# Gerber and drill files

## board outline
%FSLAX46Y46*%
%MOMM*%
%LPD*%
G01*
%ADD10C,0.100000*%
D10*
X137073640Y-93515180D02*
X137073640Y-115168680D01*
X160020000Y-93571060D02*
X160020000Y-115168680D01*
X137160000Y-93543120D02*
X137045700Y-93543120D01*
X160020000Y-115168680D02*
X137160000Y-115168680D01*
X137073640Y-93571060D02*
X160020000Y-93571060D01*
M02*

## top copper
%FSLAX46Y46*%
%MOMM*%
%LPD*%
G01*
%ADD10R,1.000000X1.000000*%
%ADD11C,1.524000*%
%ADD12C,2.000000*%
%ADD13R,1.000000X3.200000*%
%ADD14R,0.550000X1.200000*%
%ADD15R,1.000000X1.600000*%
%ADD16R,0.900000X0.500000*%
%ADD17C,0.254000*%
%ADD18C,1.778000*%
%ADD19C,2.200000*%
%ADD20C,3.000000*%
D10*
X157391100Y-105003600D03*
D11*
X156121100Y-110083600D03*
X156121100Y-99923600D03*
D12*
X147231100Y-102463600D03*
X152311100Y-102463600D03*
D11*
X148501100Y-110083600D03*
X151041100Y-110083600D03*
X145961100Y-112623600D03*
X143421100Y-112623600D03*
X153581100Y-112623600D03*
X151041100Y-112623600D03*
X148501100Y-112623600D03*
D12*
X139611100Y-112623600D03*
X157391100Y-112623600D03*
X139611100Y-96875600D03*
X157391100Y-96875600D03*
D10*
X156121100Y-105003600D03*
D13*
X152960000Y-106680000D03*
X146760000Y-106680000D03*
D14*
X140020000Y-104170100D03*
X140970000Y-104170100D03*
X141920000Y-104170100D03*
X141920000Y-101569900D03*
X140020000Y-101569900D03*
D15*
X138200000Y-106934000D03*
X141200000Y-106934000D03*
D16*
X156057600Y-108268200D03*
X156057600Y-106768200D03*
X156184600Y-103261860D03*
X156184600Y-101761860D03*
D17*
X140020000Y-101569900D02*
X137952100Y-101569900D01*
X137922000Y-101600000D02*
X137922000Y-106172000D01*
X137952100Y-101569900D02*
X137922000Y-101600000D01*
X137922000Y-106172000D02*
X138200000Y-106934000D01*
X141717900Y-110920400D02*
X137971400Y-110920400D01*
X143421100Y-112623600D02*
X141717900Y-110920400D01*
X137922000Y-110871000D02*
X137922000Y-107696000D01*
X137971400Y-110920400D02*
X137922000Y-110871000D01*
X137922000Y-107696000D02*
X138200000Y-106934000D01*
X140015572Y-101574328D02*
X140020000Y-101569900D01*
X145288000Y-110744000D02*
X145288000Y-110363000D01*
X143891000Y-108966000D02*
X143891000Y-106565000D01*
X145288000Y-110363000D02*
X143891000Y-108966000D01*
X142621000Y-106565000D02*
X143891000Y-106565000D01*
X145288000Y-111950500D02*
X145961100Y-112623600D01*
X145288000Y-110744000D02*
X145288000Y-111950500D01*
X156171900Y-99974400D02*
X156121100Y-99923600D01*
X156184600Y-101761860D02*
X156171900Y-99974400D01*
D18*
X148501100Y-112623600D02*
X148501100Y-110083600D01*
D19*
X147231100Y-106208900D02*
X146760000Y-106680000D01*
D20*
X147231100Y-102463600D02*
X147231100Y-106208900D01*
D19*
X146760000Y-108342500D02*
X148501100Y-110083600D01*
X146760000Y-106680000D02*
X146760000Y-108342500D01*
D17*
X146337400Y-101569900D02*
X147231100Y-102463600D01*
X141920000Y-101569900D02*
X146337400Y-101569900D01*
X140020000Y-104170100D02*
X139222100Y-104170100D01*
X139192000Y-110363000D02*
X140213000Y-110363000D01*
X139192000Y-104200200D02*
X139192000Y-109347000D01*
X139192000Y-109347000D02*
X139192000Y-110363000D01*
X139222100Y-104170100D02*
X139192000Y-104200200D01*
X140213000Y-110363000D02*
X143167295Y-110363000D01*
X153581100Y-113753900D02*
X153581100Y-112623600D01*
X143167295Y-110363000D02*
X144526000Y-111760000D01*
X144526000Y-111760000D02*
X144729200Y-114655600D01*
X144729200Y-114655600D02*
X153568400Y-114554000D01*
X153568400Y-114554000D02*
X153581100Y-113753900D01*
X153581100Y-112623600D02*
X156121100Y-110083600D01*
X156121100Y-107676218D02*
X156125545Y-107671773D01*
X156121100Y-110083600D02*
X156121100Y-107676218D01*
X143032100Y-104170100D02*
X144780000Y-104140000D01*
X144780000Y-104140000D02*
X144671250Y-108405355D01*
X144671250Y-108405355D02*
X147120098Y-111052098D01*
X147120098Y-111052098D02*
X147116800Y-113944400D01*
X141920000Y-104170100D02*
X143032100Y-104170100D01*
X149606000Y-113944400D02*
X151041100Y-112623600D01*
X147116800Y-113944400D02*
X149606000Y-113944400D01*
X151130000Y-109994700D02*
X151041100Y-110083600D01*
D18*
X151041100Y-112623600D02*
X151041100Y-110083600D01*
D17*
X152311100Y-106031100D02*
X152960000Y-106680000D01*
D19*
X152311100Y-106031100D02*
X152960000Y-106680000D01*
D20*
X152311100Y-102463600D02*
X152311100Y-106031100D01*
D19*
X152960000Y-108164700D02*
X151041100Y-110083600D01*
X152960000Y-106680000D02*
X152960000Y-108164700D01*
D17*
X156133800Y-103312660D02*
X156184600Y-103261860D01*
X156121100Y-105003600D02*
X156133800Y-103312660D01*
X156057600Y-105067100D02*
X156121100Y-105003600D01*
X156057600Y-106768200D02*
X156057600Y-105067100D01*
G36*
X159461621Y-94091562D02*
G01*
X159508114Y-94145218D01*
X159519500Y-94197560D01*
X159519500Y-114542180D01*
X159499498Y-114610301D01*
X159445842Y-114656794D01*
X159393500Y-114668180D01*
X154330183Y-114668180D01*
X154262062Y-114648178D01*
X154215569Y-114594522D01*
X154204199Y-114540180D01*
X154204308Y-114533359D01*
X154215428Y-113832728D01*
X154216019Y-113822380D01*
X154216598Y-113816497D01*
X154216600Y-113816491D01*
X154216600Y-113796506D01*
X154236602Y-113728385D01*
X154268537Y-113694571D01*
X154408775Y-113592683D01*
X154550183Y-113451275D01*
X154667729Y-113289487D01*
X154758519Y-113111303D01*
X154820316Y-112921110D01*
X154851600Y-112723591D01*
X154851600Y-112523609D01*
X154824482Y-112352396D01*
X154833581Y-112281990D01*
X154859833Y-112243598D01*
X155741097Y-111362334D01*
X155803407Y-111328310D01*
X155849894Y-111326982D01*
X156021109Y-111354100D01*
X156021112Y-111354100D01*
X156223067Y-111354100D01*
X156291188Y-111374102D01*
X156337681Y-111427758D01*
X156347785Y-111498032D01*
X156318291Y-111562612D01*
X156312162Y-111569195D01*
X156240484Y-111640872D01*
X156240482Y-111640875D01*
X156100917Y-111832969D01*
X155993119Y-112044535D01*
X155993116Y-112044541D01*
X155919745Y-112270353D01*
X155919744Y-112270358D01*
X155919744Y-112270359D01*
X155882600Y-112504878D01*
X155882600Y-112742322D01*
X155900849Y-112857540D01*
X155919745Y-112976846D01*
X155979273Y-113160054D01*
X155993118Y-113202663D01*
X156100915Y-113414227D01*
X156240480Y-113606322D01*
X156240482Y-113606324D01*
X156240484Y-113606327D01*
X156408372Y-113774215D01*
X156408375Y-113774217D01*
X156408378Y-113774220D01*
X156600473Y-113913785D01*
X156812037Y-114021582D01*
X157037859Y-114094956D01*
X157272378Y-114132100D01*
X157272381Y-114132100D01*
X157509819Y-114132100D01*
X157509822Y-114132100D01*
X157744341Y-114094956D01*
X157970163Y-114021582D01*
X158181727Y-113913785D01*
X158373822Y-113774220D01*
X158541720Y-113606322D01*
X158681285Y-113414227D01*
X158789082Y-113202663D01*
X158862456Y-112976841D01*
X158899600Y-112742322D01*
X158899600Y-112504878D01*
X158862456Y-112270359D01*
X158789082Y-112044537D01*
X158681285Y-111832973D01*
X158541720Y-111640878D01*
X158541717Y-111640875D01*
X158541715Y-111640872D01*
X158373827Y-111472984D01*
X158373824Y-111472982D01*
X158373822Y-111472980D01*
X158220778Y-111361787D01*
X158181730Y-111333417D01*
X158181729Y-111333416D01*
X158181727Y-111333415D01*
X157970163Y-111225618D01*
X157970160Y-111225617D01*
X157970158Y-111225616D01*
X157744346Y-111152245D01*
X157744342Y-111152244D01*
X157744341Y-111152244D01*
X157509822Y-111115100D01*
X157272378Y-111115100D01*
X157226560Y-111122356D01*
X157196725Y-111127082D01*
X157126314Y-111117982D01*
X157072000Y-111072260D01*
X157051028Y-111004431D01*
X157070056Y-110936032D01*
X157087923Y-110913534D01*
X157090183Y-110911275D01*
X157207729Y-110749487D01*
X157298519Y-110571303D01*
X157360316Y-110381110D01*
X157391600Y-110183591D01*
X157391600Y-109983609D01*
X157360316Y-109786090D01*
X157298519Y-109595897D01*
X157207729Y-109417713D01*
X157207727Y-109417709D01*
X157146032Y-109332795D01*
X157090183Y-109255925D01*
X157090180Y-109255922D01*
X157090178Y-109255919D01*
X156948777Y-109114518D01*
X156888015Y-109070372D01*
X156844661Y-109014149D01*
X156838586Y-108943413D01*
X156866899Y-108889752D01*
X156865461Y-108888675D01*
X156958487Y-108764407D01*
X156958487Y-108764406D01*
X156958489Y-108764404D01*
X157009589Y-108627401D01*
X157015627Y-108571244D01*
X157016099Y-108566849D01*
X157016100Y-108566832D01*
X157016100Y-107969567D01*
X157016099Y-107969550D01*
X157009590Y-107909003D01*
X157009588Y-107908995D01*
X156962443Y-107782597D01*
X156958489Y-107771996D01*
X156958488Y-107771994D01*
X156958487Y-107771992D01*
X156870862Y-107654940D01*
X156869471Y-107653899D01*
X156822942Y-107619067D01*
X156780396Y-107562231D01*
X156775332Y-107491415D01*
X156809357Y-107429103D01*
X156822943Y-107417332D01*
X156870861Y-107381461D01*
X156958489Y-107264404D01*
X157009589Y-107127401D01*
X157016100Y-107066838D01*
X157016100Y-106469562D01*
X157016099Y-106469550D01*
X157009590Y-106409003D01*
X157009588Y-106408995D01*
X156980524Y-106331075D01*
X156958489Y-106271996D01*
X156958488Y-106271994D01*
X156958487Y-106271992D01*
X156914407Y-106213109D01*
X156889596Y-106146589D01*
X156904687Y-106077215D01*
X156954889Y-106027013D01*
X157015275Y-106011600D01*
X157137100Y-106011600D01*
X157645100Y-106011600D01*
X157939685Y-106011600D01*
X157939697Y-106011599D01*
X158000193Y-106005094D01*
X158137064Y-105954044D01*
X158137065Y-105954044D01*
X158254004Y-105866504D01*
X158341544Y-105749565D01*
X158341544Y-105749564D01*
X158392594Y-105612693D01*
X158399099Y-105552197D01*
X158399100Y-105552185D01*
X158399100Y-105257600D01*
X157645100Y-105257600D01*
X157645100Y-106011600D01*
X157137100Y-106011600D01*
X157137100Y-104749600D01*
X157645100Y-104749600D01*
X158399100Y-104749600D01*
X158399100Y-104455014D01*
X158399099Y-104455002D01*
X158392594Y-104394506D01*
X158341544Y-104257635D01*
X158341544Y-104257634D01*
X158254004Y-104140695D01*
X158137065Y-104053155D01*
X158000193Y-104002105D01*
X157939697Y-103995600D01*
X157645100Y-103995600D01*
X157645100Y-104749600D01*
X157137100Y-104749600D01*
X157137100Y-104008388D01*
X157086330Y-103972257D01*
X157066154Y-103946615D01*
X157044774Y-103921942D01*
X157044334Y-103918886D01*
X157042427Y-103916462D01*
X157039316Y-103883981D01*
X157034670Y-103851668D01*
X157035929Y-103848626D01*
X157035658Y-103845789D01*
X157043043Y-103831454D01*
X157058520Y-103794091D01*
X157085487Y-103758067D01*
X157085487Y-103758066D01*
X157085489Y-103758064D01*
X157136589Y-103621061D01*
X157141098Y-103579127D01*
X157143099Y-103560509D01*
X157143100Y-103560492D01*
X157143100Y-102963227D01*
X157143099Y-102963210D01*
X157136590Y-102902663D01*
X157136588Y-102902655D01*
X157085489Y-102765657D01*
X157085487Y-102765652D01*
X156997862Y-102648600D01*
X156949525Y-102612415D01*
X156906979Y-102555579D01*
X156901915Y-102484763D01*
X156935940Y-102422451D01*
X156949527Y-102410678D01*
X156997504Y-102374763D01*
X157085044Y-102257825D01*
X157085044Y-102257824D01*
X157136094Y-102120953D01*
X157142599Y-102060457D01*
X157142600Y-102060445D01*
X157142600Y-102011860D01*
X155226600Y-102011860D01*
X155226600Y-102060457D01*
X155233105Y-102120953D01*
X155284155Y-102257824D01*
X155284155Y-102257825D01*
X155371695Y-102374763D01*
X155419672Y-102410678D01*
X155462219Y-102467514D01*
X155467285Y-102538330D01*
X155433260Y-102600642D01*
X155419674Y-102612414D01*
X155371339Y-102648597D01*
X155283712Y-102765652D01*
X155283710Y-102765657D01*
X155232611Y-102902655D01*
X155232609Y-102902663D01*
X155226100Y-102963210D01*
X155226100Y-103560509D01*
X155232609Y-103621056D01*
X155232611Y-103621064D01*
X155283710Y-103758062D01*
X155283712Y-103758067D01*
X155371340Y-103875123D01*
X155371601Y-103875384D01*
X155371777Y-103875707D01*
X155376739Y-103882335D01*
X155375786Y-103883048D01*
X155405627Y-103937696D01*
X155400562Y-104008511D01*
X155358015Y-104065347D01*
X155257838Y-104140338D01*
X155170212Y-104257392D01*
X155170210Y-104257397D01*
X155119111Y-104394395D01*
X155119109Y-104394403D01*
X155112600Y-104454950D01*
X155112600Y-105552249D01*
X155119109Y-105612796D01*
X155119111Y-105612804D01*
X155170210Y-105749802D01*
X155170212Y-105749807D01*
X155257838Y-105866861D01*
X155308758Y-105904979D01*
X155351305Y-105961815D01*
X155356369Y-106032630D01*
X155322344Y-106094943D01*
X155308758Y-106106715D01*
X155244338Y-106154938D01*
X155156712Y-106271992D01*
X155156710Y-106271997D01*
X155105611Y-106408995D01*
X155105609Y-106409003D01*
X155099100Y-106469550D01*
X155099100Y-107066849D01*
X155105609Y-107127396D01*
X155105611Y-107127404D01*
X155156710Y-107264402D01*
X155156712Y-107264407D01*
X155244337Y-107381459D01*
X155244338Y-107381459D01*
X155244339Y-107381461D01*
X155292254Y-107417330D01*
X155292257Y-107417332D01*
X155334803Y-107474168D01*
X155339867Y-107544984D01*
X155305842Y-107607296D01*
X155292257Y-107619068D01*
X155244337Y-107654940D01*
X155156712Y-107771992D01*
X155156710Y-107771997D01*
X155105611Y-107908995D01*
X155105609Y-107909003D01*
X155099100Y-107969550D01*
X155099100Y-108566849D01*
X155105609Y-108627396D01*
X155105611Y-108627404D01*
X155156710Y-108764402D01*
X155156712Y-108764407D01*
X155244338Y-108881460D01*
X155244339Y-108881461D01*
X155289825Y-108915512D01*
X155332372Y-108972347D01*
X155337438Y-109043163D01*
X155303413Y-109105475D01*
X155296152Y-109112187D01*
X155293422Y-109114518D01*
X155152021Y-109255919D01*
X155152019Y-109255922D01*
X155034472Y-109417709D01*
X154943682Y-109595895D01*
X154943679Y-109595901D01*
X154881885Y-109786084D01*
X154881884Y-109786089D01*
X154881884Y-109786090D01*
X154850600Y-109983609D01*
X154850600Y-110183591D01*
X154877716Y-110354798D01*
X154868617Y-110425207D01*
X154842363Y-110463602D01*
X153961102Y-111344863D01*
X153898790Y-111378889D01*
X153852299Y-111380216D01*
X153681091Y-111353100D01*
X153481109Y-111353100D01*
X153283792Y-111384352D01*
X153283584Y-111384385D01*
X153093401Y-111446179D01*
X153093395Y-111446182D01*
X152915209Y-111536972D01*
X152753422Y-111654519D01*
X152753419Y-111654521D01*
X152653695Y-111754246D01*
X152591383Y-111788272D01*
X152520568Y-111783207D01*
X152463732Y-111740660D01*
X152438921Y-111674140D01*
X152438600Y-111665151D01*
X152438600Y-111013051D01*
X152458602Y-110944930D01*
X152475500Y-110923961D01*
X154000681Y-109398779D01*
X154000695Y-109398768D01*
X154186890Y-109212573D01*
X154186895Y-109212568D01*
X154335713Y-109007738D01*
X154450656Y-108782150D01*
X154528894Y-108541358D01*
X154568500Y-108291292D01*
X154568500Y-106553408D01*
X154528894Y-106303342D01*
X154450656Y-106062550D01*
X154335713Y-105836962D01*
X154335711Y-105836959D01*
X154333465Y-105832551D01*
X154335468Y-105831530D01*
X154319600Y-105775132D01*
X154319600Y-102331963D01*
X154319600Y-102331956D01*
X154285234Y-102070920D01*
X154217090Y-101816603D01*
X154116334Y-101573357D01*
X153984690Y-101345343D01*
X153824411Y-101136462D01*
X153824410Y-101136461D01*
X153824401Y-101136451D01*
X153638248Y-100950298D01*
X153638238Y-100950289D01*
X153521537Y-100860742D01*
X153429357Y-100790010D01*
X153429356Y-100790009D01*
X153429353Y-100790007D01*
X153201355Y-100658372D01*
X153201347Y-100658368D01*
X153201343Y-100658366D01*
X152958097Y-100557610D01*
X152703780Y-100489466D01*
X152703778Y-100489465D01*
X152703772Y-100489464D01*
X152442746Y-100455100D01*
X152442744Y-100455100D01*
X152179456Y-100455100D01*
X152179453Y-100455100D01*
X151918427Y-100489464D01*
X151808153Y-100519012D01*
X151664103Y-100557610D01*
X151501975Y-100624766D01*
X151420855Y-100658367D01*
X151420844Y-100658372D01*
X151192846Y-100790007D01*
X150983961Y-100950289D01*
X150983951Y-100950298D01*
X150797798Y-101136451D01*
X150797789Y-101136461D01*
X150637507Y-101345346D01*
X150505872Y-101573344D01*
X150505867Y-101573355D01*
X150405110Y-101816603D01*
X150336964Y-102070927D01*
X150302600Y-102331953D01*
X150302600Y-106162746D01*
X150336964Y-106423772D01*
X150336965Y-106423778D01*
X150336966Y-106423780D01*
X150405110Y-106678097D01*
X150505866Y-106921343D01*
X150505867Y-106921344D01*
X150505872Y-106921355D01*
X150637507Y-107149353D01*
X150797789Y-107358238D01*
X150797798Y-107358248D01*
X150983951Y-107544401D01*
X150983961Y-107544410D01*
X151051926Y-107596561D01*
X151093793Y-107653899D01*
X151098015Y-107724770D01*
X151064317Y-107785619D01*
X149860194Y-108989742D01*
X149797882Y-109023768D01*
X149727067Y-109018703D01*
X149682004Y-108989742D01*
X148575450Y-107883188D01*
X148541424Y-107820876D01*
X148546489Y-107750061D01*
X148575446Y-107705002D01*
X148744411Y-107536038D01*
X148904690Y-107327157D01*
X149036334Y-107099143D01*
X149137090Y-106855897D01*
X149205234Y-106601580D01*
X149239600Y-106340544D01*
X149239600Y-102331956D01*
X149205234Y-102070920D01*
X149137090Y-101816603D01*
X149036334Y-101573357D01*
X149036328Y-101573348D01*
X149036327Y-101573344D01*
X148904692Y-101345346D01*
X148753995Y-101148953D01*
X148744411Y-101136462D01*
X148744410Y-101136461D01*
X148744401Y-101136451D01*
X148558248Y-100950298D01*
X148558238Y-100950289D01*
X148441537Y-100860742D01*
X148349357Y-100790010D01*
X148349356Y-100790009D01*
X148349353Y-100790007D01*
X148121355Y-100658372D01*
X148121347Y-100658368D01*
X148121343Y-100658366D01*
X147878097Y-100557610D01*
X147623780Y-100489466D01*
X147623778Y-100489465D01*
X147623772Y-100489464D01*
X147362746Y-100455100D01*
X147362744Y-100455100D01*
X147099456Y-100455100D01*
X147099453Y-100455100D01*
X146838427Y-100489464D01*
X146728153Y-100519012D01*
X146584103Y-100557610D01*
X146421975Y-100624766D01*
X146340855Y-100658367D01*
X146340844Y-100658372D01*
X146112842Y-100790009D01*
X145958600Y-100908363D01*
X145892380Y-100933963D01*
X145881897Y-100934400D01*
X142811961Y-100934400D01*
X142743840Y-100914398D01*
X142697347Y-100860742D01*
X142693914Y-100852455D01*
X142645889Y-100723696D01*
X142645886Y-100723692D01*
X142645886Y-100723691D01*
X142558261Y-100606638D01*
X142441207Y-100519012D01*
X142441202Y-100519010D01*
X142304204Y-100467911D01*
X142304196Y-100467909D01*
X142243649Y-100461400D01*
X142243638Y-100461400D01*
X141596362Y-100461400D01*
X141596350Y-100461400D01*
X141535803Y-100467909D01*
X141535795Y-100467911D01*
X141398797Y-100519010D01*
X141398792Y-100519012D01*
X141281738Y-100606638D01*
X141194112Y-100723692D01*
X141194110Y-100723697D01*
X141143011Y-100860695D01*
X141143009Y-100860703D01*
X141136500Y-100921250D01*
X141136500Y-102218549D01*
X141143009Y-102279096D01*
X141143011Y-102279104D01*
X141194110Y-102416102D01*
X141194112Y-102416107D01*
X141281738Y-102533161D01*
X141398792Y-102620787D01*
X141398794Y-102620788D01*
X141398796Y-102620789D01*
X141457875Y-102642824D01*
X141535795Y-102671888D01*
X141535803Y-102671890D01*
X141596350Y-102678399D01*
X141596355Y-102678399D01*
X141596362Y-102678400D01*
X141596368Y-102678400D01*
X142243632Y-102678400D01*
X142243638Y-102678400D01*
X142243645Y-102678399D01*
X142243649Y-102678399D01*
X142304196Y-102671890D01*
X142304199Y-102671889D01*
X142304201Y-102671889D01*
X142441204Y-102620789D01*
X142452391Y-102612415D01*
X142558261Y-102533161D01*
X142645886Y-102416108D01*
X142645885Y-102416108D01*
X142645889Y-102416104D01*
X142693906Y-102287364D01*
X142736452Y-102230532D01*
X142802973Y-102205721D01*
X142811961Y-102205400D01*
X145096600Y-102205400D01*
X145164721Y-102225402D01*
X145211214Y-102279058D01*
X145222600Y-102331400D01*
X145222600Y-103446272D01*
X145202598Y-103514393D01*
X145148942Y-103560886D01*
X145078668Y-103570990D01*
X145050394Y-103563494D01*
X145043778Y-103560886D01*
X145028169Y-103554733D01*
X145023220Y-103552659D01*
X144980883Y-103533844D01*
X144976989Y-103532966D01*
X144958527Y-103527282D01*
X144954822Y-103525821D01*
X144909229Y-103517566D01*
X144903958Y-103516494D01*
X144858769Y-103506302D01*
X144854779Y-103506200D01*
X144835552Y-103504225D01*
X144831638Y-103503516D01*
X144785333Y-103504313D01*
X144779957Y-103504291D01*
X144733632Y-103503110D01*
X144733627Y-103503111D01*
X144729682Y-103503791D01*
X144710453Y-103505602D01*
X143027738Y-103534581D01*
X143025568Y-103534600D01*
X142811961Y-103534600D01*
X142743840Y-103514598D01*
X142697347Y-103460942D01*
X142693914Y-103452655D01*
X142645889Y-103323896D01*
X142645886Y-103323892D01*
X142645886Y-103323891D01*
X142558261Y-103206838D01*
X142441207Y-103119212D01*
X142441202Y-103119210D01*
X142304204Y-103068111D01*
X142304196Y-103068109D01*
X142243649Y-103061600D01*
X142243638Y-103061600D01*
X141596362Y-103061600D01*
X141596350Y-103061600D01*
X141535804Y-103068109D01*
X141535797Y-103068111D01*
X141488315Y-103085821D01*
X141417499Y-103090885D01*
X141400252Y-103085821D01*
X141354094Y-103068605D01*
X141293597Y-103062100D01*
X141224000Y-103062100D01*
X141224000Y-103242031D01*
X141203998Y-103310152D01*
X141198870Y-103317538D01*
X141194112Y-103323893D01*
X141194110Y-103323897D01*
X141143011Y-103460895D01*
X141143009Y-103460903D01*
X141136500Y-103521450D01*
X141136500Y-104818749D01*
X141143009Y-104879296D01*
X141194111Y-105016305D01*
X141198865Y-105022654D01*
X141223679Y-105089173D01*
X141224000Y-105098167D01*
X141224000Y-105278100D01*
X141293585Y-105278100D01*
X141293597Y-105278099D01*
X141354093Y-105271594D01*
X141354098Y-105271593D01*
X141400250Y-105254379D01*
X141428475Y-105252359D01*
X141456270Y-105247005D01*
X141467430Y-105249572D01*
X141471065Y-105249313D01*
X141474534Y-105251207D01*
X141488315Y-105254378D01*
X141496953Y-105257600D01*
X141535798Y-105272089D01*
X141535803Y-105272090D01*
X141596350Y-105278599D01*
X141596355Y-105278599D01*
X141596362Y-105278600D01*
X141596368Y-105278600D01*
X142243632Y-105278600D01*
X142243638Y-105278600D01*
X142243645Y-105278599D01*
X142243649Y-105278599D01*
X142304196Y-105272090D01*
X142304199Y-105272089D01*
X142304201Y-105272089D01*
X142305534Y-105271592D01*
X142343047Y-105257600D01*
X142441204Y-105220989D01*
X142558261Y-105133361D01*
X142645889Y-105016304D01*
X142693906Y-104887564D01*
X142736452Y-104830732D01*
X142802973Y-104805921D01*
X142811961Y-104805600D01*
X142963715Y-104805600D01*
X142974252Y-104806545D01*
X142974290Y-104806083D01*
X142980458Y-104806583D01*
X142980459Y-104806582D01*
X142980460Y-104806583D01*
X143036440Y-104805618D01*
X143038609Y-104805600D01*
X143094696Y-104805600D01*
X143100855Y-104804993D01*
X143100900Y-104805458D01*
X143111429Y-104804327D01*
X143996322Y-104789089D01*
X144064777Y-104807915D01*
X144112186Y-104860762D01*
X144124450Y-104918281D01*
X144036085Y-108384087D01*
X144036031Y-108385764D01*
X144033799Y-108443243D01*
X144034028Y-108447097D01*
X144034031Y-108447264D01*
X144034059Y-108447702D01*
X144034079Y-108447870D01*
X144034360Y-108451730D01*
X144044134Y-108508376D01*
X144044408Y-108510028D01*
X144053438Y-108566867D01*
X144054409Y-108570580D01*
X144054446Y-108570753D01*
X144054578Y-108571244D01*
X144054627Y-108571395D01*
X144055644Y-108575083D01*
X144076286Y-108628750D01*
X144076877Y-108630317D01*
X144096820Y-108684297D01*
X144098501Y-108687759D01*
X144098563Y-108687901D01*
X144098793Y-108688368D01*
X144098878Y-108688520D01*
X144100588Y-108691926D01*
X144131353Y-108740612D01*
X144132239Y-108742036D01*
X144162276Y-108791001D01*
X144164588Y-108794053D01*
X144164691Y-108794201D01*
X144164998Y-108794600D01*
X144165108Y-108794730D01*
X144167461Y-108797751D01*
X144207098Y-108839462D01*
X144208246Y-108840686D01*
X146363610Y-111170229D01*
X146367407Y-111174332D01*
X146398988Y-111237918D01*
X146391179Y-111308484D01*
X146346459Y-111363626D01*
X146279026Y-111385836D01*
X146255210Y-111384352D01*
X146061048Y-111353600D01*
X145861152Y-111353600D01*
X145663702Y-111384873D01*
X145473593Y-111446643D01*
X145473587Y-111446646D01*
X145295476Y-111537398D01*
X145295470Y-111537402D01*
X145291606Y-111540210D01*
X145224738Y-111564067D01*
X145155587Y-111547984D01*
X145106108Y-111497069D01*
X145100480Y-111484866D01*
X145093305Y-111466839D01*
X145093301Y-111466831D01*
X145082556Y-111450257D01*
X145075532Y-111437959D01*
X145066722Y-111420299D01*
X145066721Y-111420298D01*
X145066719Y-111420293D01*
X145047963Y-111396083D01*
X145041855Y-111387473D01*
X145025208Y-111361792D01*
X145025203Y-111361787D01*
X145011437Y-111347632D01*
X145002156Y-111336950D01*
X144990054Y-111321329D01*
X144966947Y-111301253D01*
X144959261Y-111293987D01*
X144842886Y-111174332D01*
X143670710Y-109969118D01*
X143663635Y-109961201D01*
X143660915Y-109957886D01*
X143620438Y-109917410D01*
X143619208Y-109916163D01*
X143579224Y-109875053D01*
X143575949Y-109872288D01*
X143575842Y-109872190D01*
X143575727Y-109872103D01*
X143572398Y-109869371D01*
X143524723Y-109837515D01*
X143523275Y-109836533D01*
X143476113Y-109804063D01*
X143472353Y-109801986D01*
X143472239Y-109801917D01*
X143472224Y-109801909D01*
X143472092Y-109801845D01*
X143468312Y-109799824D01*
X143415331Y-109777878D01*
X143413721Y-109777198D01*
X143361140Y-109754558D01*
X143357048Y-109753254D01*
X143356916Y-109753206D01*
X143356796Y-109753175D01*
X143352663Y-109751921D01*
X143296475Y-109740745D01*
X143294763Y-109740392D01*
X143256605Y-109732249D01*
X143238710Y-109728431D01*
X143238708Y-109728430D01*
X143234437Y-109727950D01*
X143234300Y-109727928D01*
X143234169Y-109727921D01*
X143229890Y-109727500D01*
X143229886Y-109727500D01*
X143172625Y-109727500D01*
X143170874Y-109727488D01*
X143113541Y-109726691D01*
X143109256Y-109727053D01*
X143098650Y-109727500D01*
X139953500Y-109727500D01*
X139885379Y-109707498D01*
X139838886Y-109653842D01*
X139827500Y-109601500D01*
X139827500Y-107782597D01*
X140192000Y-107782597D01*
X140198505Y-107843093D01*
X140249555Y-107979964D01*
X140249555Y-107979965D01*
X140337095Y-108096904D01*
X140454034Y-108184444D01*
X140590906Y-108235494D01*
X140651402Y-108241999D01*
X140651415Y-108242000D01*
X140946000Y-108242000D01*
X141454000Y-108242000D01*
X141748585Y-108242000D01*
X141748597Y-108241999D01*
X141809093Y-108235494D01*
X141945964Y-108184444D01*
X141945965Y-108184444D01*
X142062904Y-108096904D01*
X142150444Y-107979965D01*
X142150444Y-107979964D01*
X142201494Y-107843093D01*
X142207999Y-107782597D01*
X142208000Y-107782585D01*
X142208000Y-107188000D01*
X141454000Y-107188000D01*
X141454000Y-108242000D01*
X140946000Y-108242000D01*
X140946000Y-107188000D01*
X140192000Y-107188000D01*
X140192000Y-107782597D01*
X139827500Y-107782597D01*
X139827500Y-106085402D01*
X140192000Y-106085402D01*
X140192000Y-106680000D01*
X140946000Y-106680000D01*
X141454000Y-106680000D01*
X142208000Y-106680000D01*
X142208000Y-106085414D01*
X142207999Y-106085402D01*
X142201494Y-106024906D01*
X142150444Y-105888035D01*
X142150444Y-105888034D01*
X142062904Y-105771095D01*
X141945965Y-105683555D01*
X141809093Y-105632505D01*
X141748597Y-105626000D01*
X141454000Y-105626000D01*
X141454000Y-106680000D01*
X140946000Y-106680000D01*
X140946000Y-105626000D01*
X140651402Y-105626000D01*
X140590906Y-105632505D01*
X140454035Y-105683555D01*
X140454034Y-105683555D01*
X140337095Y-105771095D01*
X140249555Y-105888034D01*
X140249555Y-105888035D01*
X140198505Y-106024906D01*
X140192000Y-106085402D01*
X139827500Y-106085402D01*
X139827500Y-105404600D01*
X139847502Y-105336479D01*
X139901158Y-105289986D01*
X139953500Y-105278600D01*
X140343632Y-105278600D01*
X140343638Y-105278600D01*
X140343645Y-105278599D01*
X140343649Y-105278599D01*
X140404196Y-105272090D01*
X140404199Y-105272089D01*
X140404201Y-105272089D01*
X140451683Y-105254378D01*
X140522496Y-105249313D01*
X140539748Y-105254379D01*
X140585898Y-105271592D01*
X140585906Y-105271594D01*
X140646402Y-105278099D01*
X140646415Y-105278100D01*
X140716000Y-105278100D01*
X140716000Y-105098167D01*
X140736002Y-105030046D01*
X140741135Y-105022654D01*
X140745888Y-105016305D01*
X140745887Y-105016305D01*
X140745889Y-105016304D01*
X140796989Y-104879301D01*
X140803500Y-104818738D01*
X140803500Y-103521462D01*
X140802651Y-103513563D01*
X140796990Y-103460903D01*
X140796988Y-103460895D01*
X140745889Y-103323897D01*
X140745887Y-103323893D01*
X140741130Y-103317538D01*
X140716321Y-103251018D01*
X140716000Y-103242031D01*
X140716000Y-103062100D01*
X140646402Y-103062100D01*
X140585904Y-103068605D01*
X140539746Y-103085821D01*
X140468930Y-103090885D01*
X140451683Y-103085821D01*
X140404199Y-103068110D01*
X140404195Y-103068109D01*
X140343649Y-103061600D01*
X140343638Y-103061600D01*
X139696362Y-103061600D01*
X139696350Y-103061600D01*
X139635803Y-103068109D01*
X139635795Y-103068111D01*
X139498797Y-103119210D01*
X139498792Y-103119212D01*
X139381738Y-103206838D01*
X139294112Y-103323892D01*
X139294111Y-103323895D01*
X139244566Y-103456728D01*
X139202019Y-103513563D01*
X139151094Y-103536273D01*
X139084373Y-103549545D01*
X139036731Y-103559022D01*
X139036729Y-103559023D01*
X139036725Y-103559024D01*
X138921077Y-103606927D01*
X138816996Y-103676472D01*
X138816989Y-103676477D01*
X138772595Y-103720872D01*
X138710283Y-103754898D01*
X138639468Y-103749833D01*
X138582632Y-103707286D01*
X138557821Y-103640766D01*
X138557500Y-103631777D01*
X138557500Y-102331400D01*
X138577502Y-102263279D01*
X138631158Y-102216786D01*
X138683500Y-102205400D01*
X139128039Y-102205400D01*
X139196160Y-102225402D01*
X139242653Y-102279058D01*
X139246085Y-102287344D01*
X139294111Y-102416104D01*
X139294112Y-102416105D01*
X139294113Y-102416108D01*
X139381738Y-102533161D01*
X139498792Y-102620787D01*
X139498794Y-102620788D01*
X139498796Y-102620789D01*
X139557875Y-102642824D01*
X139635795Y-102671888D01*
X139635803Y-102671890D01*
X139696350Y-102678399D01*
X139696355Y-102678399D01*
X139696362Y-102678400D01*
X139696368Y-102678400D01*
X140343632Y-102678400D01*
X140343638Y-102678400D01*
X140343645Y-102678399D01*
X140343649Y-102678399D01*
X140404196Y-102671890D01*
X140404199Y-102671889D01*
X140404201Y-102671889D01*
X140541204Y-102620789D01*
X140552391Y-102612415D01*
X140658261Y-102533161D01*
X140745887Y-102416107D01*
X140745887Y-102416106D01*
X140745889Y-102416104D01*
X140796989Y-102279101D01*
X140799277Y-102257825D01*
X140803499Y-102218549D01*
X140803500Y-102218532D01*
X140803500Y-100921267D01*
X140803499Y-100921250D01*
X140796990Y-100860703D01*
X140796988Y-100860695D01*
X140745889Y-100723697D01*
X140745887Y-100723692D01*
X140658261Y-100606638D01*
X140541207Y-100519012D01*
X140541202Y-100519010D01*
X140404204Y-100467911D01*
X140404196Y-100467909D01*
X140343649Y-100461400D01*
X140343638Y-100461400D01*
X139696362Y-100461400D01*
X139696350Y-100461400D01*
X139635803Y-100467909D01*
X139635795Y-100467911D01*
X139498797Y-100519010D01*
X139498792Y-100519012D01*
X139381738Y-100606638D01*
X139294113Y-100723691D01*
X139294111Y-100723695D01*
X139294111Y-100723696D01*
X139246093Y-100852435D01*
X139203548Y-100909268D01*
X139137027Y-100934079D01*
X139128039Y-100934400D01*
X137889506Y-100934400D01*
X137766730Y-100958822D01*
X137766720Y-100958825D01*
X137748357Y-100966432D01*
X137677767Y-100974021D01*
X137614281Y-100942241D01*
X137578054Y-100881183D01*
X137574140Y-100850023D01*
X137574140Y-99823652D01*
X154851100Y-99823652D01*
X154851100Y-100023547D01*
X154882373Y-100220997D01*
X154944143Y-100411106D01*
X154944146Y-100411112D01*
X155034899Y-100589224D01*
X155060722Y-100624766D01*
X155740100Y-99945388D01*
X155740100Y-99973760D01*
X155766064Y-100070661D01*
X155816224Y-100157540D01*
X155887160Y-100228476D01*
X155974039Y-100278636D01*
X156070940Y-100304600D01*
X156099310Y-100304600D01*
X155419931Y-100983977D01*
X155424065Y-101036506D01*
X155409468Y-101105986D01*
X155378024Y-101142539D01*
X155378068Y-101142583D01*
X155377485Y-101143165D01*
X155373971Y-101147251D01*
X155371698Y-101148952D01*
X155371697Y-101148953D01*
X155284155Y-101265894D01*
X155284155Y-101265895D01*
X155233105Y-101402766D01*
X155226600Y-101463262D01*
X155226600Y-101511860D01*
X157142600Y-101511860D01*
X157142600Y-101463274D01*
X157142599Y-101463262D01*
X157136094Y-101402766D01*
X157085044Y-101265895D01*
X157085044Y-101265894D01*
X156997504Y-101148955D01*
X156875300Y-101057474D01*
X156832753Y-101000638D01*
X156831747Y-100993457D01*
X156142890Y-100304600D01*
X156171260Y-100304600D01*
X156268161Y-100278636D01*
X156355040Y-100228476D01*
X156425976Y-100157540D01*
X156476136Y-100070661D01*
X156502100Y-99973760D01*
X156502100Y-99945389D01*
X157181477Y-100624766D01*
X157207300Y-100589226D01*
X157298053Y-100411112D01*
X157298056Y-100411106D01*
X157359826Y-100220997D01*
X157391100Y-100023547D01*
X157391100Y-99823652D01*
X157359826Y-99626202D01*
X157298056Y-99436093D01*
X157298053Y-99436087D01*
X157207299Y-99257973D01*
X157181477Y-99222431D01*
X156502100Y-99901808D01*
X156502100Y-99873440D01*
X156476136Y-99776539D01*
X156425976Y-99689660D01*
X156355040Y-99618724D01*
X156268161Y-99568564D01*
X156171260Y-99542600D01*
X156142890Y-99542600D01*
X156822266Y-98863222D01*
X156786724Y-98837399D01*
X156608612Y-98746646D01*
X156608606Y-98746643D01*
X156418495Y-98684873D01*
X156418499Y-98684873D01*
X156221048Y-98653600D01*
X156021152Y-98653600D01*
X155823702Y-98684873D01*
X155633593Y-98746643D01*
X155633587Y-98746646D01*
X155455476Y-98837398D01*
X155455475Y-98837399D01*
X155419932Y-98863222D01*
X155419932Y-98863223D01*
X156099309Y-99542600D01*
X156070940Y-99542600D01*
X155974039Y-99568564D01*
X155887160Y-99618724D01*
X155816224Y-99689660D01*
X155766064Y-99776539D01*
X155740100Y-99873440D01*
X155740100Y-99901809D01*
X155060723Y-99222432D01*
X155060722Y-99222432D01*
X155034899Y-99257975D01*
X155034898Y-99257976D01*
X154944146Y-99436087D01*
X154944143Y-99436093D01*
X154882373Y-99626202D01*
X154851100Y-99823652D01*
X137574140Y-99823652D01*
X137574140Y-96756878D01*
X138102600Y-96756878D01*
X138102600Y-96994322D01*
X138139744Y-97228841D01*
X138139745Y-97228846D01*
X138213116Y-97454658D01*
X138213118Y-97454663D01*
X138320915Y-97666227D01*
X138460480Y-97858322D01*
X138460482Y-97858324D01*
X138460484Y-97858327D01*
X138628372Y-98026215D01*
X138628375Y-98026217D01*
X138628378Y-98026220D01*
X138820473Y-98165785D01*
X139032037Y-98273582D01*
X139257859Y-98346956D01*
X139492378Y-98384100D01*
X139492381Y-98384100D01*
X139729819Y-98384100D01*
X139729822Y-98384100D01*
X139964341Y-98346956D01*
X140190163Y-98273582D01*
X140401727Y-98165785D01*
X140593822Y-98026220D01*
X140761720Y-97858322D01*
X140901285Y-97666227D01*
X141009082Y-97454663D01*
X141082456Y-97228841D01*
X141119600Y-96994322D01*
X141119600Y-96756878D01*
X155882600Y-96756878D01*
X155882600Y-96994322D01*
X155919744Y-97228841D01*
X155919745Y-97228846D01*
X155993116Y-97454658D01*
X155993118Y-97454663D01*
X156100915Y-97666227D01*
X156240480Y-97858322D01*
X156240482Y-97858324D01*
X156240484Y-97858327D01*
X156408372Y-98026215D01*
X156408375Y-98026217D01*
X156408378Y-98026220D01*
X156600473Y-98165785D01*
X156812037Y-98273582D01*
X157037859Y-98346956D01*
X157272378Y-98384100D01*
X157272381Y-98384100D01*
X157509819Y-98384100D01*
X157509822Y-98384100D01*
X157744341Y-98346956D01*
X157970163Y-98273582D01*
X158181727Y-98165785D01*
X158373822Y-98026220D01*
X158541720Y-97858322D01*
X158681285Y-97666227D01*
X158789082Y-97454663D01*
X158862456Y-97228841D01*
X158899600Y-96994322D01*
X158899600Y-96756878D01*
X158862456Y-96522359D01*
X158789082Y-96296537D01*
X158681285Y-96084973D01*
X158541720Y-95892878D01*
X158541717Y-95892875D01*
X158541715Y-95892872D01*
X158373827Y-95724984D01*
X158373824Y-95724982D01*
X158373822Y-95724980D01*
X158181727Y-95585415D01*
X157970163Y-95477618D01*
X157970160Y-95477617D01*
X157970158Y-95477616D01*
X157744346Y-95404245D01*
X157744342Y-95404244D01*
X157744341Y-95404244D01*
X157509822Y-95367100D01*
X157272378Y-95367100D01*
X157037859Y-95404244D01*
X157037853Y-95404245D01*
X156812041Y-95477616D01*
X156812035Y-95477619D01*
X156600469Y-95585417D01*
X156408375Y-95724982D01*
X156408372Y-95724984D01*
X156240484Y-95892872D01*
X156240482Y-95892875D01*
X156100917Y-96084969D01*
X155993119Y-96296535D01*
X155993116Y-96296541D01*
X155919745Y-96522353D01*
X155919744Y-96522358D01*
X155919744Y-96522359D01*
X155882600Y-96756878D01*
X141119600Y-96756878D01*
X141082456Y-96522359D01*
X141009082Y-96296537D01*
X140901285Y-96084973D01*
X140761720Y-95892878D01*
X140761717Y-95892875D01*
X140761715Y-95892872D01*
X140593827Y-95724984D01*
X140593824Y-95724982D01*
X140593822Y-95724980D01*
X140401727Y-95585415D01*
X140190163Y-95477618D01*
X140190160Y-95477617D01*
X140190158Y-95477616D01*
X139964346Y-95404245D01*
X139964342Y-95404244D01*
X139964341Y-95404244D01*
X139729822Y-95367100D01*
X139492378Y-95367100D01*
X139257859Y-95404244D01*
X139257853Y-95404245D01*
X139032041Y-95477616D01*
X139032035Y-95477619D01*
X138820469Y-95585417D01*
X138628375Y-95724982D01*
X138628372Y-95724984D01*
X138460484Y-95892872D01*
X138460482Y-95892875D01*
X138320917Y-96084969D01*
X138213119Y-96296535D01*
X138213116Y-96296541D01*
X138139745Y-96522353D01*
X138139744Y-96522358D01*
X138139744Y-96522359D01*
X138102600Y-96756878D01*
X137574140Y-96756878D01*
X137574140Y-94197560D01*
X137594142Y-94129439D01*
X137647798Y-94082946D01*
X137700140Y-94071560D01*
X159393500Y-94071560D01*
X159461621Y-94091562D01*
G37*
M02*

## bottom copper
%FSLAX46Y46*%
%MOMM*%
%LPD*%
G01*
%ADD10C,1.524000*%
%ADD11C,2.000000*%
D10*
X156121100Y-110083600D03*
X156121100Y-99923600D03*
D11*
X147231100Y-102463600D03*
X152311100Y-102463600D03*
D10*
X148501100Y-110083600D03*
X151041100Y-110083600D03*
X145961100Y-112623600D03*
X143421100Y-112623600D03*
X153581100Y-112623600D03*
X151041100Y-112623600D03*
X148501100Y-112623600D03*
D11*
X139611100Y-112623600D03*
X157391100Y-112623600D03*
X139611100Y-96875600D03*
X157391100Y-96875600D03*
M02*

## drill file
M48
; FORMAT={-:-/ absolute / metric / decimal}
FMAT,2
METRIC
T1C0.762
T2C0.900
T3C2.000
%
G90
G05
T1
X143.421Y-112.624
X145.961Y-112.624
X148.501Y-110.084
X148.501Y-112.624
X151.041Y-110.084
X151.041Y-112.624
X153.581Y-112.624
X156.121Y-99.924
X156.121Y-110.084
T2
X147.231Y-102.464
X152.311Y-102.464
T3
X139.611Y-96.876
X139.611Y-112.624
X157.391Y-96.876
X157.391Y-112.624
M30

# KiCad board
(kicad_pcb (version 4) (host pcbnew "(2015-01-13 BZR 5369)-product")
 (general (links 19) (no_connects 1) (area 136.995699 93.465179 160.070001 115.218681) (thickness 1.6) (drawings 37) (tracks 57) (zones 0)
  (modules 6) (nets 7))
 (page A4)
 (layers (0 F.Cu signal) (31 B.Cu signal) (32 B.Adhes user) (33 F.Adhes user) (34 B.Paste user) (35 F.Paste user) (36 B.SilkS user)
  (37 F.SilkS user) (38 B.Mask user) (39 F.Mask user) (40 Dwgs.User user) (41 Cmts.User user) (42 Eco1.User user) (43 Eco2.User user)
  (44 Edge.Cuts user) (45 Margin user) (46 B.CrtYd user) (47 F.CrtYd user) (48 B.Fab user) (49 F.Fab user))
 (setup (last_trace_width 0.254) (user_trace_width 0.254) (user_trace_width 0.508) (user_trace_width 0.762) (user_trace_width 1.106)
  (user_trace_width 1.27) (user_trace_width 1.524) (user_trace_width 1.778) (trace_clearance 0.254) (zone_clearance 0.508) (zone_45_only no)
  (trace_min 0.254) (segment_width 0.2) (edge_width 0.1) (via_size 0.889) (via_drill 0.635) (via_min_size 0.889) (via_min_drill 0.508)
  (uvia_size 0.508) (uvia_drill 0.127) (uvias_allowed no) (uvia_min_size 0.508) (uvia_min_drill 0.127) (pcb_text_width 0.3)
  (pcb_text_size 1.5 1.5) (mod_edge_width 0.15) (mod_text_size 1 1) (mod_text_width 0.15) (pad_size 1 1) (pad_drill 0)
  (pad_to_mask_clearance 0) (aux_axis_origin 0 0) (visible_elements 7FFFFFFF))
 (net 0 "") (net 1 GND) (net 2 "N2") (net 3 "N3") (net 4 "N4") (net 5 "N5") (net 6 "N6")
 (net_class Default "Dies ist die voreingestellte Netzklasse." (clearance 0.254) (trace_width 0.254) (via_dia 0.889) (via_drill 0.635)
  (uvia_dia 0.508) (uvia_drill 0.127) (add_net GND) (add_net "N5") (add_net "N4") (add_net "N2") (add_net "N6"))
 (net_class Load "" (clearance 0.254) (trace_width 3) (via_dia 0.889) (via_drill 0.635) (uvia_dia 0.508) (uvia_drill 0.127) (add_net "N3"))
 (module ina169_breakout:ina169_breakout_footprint (layer F.Cu) (at 148.5011 105.0036)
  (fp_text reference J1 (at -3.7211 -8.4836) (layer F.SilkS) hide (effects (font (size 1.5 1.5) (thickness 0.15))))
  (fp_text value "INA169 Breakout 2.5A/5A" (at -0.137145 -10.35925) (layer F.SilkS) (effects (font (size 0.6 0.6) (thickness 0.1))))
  (pad 2 smd rect (at 8.89 0) (size 1 1) (layers F.Cu F.Paste F.Mask) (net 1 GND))
  (pad 5 thru_hole circle (at 7.62 5.08) (size 1.524 1.524) (drill 0.762) (layers *.Cu *.Mask F.SilkS) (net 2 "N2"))
  (pad 2 thru_hole circle (at 7.62 -5.08) (size 1.524 1.524) (drill 0.762) (layers *.Cu *.Mask F.SilkS) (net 1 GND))
  (pad 3 thru_hole circle (at -1.27 -2.54) (size 2 2) (drill 0.9) (layers *.Cu *.Mask F.SilkS) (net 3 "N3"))
  (pad 4 thru_hole circle (at 3.81 -2.54) (size 2 2) (drill 0.9) (layers *.Cu *.Mask F.SilkS) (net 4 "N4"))
  (pad 3 thru_hole circle (at 0 5.08) (size 1.524 1.524) (drill 0.762) (layers *.Cu *.Mask F.SilkS) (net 3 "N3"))
  (pad 4 thru_hole circle (at 2.54 5.08) (size 1.524 1.524) (drill 0.762) (layers *.Cu *.Mask F.SilkS) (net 4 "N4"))
  (pad 2 thru_hole circle (at -2.54 7.62) (size 1.524 1.524) (drill 0.762) (layers *.Cu *.Mask F.SilkS) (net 1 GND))
  (pad 1 thru_hole circle (at -5.08 7.62) (size 1.524 1.524) (drill 0.762) (layers *.Cu *.Mask F.SilkS) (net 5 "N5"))
  (pad 5 thru_hole circle (at 5.08 7.62) (size 1.524 1.524) (drill 0.762) (layers *.Cu *.Mask F.SilkS) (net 2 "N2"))
  (pad 4 thru_hole circle (at 2.54 7.62) (size 1.524 1.524) (drill 0.762) (layers *.Cu *.Mask F.SilkS) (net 4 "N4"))
  (pad 3 thru_hole circle (at 0 7.62) (size 1.524 1.524) (drill 0.762) (layers *.Cu *.Mask F.SilkS) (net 3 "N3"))
  (pad "" thru_hole circle (at -8.89 7.62) (size 2 2) (drill 2) (layers *.Cu *.Mask F.SilkS))
  (pad "" thru_hole circle (at 8.89 7.62) (size 2 2) (drill 2) (layers *.Cu *.Mask F.SilkS))
  (pad "" thru_hole circle (at -8.89 -8.128) (size 2 2) (drill 2) (layers *.Cu *.Mask F.SilkS))
  (pad "" thru_hole circle (at 8.89 -8.128) (size 2 2) (drill 2) (layers *.Cu *.Mask F.SilkS))
  (pad 6 smd rect (at 7.62 0) (size 1 1) (layers F.Cu F.Paste F.Mask)))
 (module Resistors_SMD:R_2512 (layer F.Cu) (at 149.86 106.68 180)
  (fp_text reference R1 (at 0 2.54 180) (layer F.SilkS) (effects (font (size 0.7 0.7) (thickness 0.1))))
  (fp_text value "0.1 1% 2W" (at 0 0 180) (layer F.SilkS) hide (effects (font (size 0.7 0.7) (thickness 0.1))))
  (pad 1 smd rect (at -3.1 0 180) (size 1 3.2) (layers F.Cu F.Paste F.Mask) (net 4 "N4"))
  (pad 2 smd rect (at 3.1 0 180) (size 1 3.2) (layers F.Cu F.Paste F.Mask) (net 3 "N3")))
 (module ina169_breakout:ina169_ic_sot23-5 (layer F.Cu) (at 140.97 102.87)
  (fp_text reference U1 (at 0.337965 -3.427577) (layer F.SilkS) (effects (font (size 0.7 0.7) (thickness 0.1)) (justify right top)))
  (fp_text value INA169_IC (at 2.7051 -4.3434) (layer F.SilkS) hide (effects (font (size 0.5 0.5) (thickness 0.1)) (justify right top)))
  (pad 1 smd rect (at -0.95 1.3001) (size 0.55 1.2) (layers F.Cu F.Paste F.Mask) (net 2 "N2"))
  (pad 2 smd rect (at 0 1.3001) (size 0.55 1.2) (layers F.Cu F.Paste F.Mask) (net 1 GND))
  (pad 3 smd rect (at 0.95 1.3001) (size 0.55 1.2) (layers F.Cu F.Paste F.Mask) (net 4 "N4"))
  (pad 4 smd rect (at 0.95 -1.3001) (size 0.55 1.2) (layers F.Cu F.Paste F.Mask) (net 3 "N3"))
  (pad 5 smd rect (at -0.95 -1.3001) (size 0.55 1.2) (layers F.Cu F.Paste F.Mask) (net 5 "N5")))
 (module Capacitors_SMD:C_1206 (layer F.Cu) (at 139.7 106.934)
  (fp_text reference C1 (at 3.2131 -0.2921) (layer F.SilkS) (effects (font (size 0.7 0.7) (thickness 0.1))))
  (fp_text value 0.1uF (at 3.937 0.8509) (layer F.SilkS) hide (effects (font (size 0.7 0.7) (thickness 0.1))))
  (pad 1 smd rect (at -1.5 0) (size 1 1.6) (layers F.Cu F.Paste F.Mask) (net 5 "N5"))
  (pad 2 smd rect (at 1.5 0) (size 1 1.6) (layers F.Cu F.Paste F.Mask) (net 1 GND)))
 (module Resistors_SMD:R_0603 (layer F.Cu) (at 156.0576 107.5182 90)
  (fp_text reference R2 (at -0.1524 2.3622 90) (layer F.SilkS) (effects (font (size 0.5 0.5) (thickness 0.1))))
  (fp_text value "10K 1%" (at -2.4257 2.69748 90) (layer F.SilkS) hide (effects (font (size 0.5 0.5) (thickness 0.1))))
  (pad 1 smd rect (at -0.75 0 90) (size 0.5 0.9) (layers F.Cu F.Paste F.Mask) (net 2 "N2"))
  (pad 2 smd rect (at 0.75 0 90) (size 0.5 0.9) (layers F.Cu F.Paste F.Mask) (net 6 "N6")))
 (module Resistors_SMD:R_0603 (layer F.Cu) (at 156.1846 102.51186 90)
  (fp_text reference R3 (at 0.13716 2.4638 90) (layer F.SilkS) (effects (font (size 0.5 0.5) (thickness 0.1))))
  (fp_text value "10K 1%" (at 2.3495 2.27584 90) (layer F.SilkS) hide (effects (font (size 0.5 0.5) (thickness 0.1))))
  (pad 1 smd rect (at -0.75 0 90) (size 0.5 0.9) (layers F.Cu F.Paste F.Mask) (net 6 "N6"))
  (pad 2 smd rect (at 0.75 0 90) (size 0.5 0.9) (layers F.Cu F.Paste F.Mask) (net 1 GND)))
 (gr_line (start 137.07364 93.51518) (end 137.07364 115.16868) (angle 90) (layer Edge.Cuts) (width 0.1))
 (gr_line (start 160.02 93.57106) (end 160.02 115.16868) (angle 90) (layer Edge.Cuts) (width 0.1))
 (gr_line (start 137.16 93.54312) (end 137.0457 93.54312) (angle 90) (layer Edge.Cuts) (width 0.1))
 (gr_line (start 160.02 115.16868) (end 137.16 115.16868) (angle 90) (layer Edge.Cuts) (width 0.1))
 (gr_line (start 137.07364 93.57106) (end 160.02 93.57106) (angle 90) (layer Edge.Cuts) (width 0.1))
 (segment (start 140.02 101.5699) (end 137.9521 101.5699) (width 0.254) (layer F.Cu) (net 5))
 (segment (start 137.922 101.6) (end 137.922 106.172) (width 0.254) (layer F.Cu) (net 5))
 (segment (start 137.9521 101.5699) (end 137.922 101.6) (width 0.254) (layer F.Cu) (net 5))
 (segment (start 137.922 106.172) (end 138.2 106.934) (width 0.254) (layer F.Cu) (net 5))
 (segment (start 141.7179 110.9204) (end 137.9714 110.9204) (width 0.254) (layer F.Cu) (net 5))
 (segment (start 143.4211 112.6236) (end 141.7179 110.9204) (width 0.254) (layer F.Cu) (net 5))
 (segment (start 137.922 110.871) (end 137.922 107.696) (width 0.254) (layer F.Cu) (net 5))
 (segment (start 137.9714 110.9204) (end 137.922 110.871) (width 0.254) (layer F.Cu) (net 5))
 (segment (start 137.922 107.696) (end 138.2 106.934) (width 0.254) (layer F.Cu) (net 5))
 (segment (start 140.015572 101.574328) (end 140.02 101.5699) (width 0.254) (layer F.Cu) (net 5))
 (segment (start 145.288 110.744) (end 145.288 110.363) (width 0.254) (layer F.Cu) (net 1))
 (segment (start 143.891 108.966) (end 143.891 106.565) (width 0.254) (layer F.Cu) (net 1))
 (segment (start 145.288 110.363) (end 143.891 108.966) (width 0.254) (layer F.Cu) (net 1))
 (segment (start 142.621 106.565) (end 143.891 106.565) (width 0.254) (layer F.Cu) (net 1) (status 10))
 (segment (start 145.288 111.9505) (end 145.9611 112.6236) (width 0.254) (layer F.Cu) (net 1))
 (segment (start 145.288 110.744) (end 145.288 111.9505) (width 0.254) (layer F.Cu) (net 1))
 (segment (start 156.1719 99.9744) (end 156.1211 99.9236) (width 0.254) (layer F.Cu) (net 1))
 (segment (start 156.1846 101.76186) (end 156.1719 99.9744) (width 0.254) (layer F.Cu) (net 1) (status 10))
 (segment (start 148.5011 112.6236) (end 148.5011 110.0836) (width 1.778) (layer F.Cu) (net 3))
 (segment (start 147.2311 106.2089) (end 146.76 106.68) (width 2.2) (layer F.Cu) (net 3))
 (segment (start 147.2311 102.4636) (end 147.2311 106.2089) (width 3) (layer F.Cu) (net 3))
 (segment (start 146.76 108.3425) (end 148.5011 110.0836) (width 2.2) (layer F.Cu) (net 3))
 (segment (start 146.76 106.68) (end 146.76 108.3425) (width 2.2) (layer F.Cu) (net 3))
 (segment (start 146.3374 101.5699) (end 147.2311 102.4636) (width 0.254) (layer F.Cu) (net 3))
 (segment (start 141.92 101.5699) (end 146.3374 101.5699) (width 0.254) (layer F.Cu) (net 3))
 (segment (start 140.02 104.1701) (end 139.2221 104.1701) (width 0.254) (layer F.Cu) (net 2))
 (segment (start 139.192 110.363) (end 140.213 110.363) (width 0.254) (layer F.Cu) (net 2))
 (segment (start 139.192 104.2002) (end 139.192 109.347) (width 0.254) (layer F.Cu) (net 2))
 (segment (start 139.192 109.347) (end 139.192 110.363) (width 0.254) (layer F.Cu) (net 2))
 (segment (start 139.2221 104.1701) (end 139.192 104.2002) (width 0.254) (layer F.Cu) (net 2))
 (segment (start 140.213 110.363) (end 143.167295 110.363) (width 0.254) (layer F.Cu) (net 2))
 (segment (start 153.5811 113.7539) (end 153.5811 112.6236) (width 0.254) (layer F.Cu) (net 2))
 (segment (start 143.167295 110.363) (end 144.526 111.76) (width 0.254) (layer F.Cu) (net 2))
 (segment (start 144.526 111.76) (end 144.7292 114.6556) (width 0.254) (layer F.Cu) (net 2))
 (segment (start 144.7292 114.6556) (end 153.5684 114.554) (width 0.254) (layer F.Cu) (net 2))
 (segment (start 153.5684 114.554) (end 153.5811 113.7539) (width 0.254) (layer F.Cu) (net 2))
 (segment (start 153.5811 112.6236) (end 156.1211 110.0836) (width 0.254) (layer F.Cu) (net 2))
 (segment (start 156.1211 107.676218) (end 156.125545 107.671773) (width 0.254) (layer F.Cu) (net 2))
 (segment (start 156.1211 110.0836) (end 156.1211 107.676218) (width 0.254) (layer F.Cu) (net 2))
 (segment (start 143.0321 104.1701) (end 144.78 104.14) (width 0.254) (layer F.Cu) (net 4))
 (segment (start 144.78 104.14) (end 144.67125 108.405355) (width 0.254) (layer F.Cu) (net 4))
 (segment (start 144.67125 108.405355) (end 147.120098 111.052098) (width 0.254) (layer F.Cu) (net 4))
 (segment (start 147.120098 111.052098) (end 147.1168 113.9444) (width 0.254) (layer F.Cu) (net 4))
 (segment (start 141.92 104.1701) (end 143.0321 104.1701) (width 0.254) (layer F.Cu) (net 4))
 (segment (start 149.606 113.9444) (end 151.0411 112.6236) (width 0.254) (layer F.Cu) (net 4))
 (segment (start 147.1168 113.9444) (end 149.606 113.9444) (width 0.254) (layer F.Cu) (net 4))
 (segment (start 151.13 109.9947) (end 151.0411 110.0836) (width 0.254) (layer F.Cu) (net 4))
 (segment (start 151.0411 112.6236) (end 151.0411 110.0836) (width 1.778) (layer F.Cu) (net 4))
 (segment (start 152.3111 106.0311) (end 152.96 106.68) (width 0.254) (layer F.Cu) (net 4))
 (segment (start 152.3111 106.0311) (end 152.96 106.68) (width 2.2) (layer F.Cu) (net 4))
 (segment (start 152.3111 102.4636) (end 152.3111 106.0311) (width 3) (layer F.Cu) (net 4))
 (segment (start 152.96 108.1647) (end 151.0411 110.0836) (width 2.2) (layer F.Cu) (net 4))
 (segment (start 152.96 106.68) (end 152.96 108.1647) (width 2.2) (layer F.Cu) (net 4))
 (segment (start 156.1338 103.31266) (end 156.1846 103.26186) (width 0.254) (layer F.Cu) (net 6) (status 30))
 (segment (start 156.1211 105.0036) (end 156.1338 103.31266) (width 0.254) (layer F.Cu) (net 6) (status 20))
 (segment (start 156.0576 105.0671) (end 156.1211 105.0036) (width 0.254) (layer F.Cu) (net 6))
 (segment (start 156.0576 106.7682) (end 156.0576 105.0671) (width 0.254) (layer F.Cu) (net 6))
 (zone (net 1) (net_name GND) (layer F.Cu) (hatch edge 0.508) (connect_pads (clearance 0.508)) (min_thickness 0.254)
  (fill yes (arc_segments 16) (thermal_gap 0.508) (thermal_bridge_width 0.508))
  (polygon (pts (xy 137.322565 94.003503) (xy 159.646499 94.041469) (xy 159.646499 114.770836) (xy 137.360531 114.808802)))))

